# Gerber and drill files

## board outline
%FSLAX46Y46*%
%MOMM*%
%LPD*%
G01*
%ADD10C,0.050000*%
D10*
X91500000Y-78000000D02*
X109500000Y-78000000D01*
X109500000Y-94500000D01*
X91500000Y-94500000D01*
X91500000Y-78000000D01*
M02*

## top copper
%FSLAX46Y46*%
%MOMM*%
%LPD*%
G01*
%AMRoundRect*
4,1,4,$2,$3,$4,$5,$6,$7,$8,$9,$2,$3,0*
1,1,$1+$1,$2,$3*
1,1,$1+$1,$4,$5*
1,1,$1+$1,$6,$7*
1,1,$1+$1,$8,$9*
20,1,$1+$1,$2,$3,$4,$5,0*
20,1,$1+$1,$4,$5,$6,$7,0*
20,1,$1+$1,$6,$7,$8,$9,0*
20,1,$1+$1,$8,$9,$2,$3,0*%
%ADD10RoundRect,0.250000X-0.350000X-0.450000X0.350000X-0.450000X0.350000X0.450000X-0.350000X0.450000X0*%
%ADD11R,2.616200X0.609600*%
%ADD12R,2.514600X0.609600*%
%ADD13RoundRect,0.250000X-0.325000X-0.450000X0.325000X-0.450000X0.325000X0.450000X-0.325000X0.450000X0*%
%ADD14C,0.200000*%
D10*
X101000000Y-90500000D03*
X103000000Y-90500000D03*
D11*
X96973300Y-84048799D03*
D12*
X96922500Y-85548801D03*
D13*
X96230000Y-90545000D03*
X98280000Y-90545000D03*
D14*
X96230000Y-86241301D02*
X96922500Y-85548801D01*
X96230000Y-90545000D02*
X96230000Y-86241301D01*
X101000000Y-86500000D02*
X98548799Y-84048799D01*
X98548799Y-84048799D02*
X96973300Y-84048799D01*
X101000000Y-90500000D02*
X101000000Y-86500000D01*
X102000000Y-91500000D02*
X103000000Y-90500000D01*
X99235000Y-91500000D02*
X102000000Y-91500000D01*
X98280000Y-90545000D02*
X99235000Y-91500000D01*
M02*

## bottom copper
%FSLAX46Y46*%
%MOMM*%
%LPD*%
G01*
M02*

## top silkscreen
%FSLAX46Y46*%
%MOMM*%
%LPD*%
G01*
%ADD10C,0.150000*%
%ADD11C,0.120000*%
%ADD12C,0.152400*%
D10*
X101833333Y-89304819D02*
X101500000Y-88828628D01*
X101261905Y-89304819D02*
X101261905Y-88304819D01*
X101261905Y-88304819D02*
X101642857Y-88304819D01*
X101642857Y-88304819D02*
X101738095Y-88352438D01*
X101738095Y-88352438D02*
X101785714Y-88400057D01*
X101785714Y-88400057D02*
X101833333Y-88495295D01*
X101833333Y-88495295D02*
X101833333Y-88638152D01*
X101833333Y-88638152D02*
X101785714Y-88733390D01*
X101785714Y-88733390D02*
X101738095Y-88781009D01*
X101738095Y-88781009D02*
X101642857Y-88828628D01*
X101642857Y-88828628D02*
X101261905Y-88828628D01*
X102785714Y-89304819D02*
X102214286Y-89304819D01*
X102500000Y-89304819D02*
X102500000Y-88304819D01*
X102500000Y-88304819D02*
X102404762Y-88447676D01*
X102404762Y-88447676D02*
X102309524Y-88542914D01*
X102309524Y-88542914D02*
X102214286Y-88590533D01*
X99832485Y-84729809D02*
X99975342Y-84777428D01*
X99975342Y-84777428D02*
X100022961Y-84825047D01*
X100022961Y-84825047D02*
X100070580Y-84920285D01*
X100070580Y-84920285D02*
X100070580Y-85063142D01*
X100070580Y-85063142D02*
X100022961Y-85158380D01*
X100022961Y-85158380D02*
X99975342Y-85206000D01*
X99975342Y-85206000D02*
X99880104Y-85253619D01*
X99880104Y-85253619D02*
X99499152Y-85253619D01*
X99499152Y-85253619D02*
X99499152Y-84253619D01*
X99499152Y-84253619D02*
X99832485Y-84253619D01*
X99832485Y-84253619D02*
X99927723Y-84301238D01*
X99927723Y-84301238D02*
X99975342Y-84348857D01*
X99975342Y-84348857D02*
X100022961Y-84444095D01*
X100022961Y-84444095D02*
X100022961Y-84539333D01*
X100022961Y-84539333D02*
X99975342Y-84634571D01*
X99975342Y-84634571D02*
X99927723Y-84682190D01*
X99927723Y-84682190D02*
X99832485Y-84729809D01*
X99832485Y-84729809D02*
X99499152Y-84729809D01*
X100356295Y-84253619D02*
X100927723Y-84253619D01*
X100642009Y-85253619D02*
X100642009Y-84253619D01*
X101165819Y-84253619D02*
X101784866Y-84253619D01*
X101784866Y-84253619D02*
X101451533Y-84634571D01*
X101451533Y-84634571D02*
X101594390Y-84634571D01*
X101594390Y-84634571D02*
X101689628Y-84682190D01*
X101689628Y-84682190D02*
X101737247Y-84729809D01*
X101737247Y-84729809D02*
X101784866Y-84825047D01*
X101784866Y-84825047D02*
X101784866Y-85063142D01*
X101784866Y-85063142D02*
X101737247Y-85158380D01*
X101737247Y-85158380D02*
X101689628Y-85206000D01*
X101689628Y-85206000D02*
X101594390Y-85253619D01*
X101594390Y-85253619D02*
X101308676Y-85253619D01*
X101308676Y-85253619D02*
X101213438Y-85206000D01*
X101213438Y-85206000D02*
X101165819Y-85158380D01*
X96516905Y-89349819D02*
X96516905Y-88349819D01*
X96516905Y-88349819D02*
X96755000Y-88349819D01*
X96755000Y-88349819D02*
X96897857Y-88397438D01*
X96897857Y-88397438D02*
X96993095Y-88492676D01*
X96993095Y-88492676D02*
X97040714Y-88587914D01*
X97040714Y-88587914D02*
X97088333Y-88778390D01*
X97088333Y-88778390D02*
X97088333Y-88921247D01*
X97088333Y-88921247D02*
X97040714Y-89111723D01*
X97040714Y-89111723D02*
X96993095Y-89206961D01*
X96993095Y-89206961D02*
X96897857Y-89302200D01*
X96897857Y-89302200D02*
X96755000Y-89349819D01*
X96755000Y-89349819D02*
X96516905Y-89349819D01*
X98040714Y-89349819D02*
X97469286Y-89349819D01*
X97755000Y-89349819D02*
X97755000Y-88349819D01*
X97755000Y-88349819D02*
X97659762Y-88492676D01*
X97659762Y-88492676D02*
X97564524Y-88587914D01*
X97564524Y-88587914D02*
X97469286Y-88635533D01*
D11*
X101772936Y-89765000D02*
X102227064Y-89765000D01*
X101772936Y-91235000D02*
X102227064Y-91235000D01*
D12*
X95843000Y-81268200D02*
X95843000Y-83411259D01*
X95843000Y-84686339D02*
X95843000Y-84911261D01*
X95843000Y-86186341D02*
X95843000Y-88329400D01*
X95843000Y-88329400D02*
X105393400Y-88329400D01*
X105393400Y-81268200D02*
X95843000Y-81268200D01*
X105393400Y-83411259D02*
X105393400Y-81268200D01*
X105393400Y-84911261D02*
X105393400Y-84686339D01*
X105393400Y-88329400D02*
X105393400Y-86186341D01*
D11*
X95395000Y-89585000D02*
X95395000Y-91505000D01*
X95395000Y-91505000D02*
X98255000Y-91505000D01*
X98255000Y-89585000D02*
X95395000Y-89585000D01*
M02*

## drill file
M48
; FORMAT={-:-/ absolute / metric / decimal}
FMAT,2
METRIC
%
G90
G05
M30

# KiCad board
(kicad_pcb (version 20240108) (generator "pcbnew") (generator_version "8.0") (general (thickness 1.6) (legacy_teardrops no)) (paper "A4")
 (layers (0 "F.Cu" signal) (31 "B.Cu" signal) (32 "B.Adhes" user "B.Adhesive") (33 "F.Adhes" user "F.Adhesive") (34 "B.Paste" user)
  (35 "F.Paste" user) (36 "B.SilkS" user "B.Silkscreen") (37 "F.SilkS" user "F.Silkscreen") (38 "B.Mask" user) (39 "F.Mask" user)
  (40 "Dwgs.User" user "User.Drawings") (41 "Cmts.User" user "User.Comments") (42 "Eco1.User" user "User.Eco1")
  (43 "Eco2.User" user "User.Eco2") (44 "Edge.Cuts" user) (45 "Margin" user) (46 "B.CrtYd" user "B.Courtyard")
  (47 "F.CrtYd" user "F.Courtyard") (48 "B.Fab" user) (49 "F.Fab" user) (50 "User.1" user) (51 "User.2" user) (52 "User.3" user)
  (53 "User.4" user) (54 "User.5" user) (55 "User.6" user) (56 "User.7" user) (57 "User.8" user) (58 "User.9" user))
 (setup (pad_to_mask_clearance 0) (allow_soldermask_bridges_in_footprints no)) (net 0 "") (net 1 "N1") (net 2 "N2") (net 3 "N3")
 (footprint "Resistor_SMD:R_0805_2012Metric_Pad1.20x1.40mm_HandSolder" (layer "F.Cu") (at 102 90.5)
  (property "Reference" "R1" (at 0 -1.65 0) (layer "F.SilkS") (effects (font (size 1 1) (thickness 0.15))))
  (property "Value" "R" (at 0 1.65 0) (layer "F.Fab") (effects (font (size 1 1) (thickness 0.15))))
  (fp_line (start -0.227064 -0.735) (end 0.227064 -0.735) (stroke (width 0.12) (type solid)) (layer "F.SilkS"))
  (fp_line (start -0.227064 0.735) (end 0.227064 0.735) (stroke (width 0.12) (type solid)) (layer "F.SilkS"))
  (pad "1" smd roundrect (at -1 0) (size 1.2 1.4) (layers "F.Cu" "F.Paste" "F.Mask") (roundrect_rratio 0.208333) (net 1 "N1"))
  (pad "2" smd roundrect (at 1 0) (size 1.2 1.4) (layers "F.Cu" "F.Paste" "F.Mask") (roundrect_rratio 0.208333) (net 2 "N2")))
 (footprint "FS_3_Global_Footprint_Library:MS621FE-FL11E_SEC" (layer "F.Cu") (at 100.6182 84.7988)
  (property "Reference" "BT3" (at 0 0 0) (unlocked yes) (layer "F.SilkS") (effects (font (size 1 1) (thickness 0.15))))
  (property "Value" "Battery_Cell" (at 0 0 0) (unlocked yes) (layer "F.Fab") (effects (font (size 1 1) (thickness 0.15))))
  (fp_line (start -4.7752 -3.5306) (end -4.7752 -1.387541) (stroke (width 0.1524) (type solid)) (layer "F.SilkS"))
  (fp_line (start -4.7752 -0.112461) (end -4.7752 0.112461) (stroke (width 0.1524) (type solid)) (layer "F.SilkS"))
  (fp_line (start -4.7752 1.387541) (end -4.7752 3.5306) (stroke (width 0.1524) (type solid)) (layer "F.SilkS"))
  (fp_line (start -4.7752 3.5306) (end 4.7752 3.5306) (stroke (width 0.1524) (type solid)) (layer "F.SilkS"))
  (fp_line (start 4.7752 -3.5306) (end -4.7752 -3.5306) (stroke (width 0.1524) (type solid)) (layer "F.SilkS"))
  (fp_line (start 4.7752 -1.387541) (end 4.7752 -3.5306) (stroke (width 0.1524) (type solid)) (layer "F.SilkS"))
  (fp_line (start 4.7752 0.112461) (end 4.7752 -0.112461) (stroke (width 0.1524) (type solid)) (layer "F.SilkS"))
  (fp_line (start 4.7752 3.5306) (end 4.7752 1.387541) (stroke (width 0.1524) (type solid)) (layer "F.SilkS"))
  (pad "1" smd rect (at -3.6449 -0.750001) (size 2.6162 0.6096) (layers "F.Cu" "F.Paste" "F.Mask") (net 1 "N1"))
  (pad "2" smd rect (at -3.6957 0.750001) (size 2.5146 0.6096) (layers "F.Cu" "F.Paste" "F.Mask") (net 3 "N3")))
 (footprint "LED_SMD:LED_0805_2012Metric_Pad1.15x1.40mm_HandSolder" (layer "F.Cu") (at 97.255 90.545)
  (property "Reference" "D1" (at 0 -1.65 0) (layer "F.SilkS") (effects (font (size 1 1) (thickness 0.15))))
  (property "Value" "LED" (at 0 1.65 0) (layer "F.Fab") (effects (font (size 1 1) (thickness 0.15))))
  (fp_line (start -1.86 -0.96) (end -1.86 0.96) (stroke (width 0.12) (type solid)) (layer "F.SilkS"))
  (fp_line (start -1.86 0.96) (end 1 0.96) (stroke (width 0.12) (type solid)) (layer "F.SilkS"))
  (fp_line (start 1 -0.96) (end -1.86 -0.96) (stroke (width 0.12) (type solid)) (layer "F.SilkS"))
  (pad "1" smd roundrect (at -1.025 0) (size 1.15 1.4) (layers "F.Cu" "F.Paste" "F.Mask") (roundrect_rratio 0.217391) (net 3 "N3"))
  (pad "2" smd roundrect (at 1.025 0) (size 1.15 1.4) (layers "F.Cu" "F.Paste" "F.Mask") (roundrect_rratio 0.217391) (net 2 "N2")))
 (gr_rect (start 91.5 78) (end 109.5 94.5) (stroke (width 0.05) (type default)) (fill none) (layer "Edge.Cuts"))
 (segment (start 96.23 86.241301) (end 96.9225 85.548801) (width 0.2) (layer "F.Cu") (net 3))
 (segment (start 96.23 90.545) (end 96.23 86.241301) (width 0.2) (layer "F.Cu") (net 3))
 (segment (start 101 86.5) (end 98.548799 84.048799) (width 0.2) (layer "F.Cu") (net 1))
 (segment (start 98.548799 84.048799) (end 96.9733 84.048799) (width 0.2) (layer "F.Cu") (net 1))
 (segment (start 101 90.5) (end 101 86.5) (width 0.2) (layer "F.Cu") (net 1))
 (segment (start 102 91.5) (end 103 90.5) (width 0.2) (layer "F.Cu") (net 2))
 (segment (start 99.235 91.5) (end 102 91.5) (width 0.2) (layer "F.Cu") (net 2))
 (segment (start 98.28 90.545) (end 99.235 91.5) (width 0.2) (layer "F.Cu") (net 2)))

